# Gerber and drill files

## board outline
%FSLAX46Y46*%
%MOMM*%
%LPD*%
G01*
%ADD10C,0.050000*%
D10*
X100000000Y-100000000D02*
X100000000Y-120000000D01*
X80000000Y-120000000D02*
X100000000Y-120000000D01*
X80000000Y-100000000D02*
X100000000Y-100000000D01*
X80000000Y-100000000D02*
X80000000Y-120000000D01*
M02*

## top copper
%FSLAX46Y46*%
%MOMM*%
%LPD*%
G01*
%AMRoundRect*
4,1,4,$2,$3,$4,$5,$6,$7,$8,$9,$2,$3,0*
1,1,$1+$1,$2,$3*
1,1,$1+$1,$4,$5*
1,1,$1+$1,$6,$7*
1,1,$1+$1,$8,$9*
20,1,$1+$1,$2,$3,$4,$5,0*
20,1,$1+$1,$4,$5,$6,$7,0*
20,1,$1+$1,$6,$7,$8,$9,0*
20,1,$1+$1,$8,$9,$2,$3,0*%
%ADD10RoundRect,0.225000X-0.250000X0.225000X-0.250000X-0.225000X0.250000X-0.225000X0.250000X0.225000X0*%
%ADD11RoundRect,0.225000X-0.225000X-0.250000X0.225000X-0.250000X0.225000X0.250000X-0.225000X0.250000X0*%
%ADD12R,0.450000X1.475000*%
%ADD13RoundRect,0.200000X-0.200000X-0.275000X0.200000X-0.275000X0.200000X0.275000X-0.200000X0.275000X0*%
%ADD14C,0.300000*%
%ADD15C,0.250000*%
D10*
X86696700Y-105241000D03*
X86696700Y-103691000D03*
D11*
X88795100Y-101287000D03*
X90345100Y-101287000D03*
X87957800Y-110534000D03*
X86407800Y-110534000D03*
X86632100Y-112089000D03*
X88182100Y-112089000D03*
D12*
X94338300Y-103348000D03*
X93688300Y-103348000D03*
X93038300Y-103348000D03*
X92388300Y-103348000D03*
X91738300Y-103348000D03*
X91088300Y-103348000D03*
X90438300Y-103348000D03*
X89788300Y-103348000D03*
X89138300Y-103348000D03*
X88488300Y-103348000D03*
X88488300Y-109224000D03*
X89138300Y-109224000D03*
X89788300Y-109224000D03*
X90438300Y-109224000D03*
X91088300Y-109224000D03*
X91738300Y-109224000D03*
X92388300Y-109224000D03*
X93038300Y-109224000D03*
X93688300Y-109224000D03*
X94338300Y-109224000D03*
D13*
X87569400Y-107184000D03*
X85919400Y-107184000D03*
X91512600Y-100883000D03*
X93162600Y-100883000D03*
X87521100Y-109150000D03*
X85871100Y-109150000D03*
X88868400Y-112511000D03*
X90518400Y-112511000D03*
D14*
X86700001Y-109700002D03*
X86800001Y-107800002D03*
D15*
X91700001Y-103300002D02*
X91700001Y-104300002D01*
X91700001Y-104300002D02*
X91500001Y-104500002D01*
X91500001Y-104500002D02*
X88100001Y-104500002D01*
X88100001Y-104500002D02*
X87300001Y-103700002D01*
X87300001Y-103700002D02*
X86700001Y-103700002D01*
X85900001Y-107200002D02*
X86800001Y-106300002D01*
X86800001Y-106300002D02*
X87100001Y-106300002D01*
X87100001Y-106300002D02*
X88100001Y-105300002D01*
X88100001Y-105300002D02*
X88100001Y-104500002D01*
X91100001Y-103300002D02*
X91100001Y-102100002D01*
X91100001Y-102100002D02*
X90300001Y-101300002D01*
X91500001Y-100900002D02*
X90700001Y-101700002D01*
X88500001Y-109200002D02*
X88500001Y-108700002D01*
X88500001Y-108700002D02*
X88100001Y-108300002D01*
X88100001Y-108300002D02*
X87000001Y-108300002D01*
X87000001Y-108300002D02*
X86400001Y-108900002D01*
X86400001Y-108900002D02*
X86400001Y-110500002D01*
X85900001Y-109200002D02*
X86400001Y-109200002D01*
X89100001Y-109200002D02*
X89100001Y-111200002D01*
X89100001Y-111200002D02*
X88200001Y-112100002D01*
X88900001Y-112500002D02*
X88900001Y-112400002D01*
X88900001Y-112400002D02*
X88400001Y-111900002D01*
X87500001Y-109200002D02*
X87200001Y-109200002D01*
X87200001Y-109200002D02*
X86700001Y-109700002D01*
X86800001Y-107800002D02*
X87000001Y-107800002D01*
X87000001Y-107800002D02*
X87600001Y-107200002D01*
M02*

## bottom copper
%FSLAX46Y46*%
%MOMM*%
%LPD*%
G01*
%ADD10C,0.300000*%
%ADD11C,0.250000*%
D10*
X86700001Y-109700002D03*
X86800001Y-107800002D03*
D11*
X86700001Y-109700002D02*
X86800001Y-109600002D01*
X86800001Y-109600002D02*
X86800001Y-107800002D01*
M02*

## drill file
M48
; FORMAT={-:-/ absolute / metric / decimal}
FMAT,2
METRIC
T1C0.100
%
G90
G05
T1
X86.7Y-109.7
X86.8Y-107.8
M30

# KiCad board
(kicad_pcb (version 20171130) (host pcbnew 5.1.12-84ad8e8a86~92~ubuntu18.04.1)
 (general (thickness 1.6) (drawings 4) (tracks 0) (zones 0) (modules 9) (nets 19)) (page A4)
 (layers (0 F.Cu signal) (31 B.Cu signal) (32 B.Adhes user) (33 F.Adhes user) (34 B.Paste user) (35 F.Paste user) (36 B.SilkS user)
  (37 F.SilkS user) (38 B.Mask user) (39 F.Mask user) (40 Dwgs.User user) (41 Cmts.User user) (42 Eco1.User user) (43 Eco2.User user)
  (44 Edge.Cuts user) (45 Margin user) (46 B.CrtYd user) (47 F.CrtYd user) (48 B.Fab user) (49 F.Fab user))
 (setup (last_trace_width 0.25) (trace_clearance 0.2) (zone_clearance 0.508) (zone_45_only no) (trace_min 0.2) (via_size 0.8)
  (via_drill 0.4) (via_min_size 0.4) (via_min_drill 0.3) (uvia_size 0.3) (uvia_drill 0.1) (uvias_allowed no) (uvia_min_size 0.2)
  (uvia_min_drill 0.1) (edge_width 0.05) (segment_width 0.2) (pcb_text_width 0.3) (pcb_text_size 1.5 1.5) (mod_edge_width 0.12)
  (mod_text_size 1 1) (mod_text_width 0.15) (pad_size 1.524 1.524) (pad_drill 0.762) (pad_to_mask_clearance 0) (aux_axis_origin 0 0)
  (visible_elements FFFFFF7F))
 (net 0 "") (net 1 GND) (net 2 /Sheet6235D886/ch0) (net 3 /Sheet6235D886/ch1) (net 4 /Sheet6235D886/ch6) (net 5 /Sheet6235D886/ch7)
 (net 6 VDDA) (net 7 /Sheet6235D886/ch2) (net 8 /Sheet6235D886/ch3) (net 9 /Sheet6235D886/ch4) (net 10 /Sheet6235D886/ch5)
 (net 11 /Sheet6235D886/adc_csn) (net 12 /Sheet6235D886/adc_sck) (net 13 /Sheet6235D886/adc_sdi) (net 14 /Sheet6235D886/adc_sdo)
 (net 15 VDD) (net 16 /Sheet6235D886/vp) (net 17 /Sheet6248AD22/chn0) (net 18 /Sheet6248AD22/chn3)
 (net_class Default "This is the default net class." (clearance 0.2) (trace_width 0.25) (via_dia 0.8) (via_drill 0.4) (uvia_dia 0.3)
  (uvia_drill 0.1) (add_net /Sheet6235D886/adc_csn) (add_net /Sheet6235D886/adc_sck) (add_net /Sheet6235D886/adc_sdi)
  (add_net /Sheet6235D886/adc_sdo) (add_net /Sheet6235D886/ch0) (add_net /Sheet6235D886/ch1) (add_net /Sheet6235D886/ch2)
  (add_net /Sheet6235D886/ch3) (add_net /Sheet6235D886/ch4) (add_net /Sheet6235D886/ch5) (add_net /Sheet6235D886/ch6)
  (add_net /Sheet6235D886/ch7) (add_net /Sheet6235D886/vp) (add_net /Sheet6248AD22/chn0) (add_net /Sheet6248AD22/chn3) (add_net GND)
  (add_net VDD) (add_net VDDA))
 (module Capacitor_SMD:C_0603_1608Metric (layer F.Cu) (at 86.696700 104.466000 270.000000)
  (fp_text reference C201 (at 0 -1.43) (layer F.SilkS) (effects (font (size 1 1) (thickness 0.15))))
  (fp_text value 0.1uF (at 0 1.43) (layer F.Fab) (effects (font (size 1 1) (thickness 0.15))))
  (pad 2 smd roundrect (at 0.775 0 270.000000) (size 0.9 0.95) (layers F.Cu F.Mask F.Paste) (roundrect_rratio 0.25) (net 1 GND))
  (pad 1 smd roundrect (at -0.775 0 270.000000) (size 0.9 0.95) (layers F.Cu F.Mask F.Paste) (roundrect_rratio 0.25)
   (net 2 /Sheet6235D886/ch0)))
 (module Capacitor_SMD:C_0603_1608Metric (layer F.Cu) (at 89.570100 101.287000)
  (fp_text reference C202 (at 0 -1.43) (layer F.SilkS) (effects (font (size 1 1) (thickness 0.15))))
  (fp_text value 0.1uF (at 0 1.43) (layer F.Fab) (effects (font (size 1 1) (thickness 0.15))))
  (pad 1 smd roundrect (at -0.775 0) (size 0.9 0.95) (layers F.Cu F.Mask F.Paste) (roundrect_rratio 0.25) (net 1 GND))
  (pad 2 smd roundrect (at 0.775 0) (size 0.9 0.95) (layers F.Cu F.Mask F.Paste) (roundrect_rratio 0.25) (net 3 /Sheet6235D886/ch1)))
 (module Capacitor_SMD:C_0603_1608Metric (layer F.Cu) (at 87.182800 110.534000)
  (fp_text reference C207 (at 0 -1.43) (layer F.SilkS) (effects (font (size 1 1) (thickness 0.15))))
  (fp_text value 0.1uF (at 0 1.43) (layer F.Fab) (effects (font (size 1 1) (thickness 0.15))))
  (pad 2 smd roundrect (at 0.775 0) (size 0.9 0.95) (layers F.Cu F.Mask F.Paste) (roundrect_rratio 0.25) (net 1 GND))
  (pad 1 smd roundrect (at -0.775 0) (size 0.9 0.95) (layers F.Cu F.Mask F.Paste) (roundrect_rratio 0.25) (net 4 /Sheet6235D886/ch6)))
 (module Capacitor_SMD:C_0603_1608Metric (layer F.Cu) (at 87.407100 112.089000)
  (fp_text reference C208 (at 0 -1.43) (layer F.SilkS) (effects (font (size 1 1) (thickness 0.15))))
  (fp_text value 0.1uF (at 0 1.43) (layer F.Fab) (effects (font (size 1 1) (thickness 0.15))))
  (pad 1 smd roundrect (at -0.775 0) (size 0.9 0.95) (layers F.Cu F.Mask F.Paste) (roundrect_rratio 0.25) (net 1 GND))
  (pad 2 smd roundrect (at 0.775 0) (size 0.9 0.95) (layers F.Cu F.Mask F.Paste) (roundrect_rratio 0.25) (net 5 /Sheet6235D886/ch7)))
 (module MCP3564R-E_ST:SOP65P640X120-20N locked (layer F.Cu) (at 91.413300 106.286000 270.000000)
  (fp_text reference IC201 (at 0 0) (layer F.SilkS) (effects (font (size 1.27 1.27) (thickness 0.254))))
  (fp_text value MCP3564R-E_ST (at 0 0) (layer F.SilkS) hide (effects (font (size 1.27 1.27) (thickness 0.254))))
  (pad 1 smd rect (at -2.938 -2.925) (size 0.45 1.475) (layers F.Cu F.Mask F.Paste) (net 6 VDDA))
  (pad 2 smd rect (at -2.938 -2.275) (size 0.45 1.475) (layers F.Cu F.Mask F.Paste) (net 1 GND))
  (pad 3 smd rect (at -2.938 -1.625) (size 0.45 1.475) (layers F.Cu F.Mask F.Paste) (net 1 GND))
  (pad 4 smd rect (at -2.938 -0.975) (size 0.45 1.475) (layers F.Cu F.Mask F.Paste))
  (pad 5 smd rect (at -2.938 -0.325) (size 0.45 1.475) (layers F.Cu F.Mask F.Paste) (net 2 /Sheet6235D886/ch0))
  (pad 6 smd rect (at -2.938 0.325) (size 0.45 1.475) (layers F.Cu F.Mask F.Paste) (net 3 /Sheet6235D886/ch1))
  (pad 7 smd rect (at -2.938 0.975) (size 0.45 1.475) (layers F.Cu F.Mask F.Paste) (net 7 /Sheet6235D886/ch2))
  (pad 8 smd rect (at -2.938 1.625) (size 0.45 1.475) (layers F.Cu F.Mask F.Paste) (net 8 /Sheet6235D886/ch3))
  (pad 9 smd rect (at -2.938 2.275) (size 0.45 1.475) (layers F.Cu F.Mask F.Paste) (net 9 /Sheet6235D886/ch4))
  (pad 10 smd rect (at -2.938 2.925) (size 0.45 1.475) (layers F.Cu F.Mask F.Paste) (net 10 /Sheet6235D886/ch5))
  (pad 11 smd rect (at 2.938 2.925) (size 0.45 1.475) (layers F.Cu F.Mask F.Paste) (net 4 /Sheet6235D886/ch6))
  (pad 12 smd rect (at 2.938 2.275) (size 0.45 1.475) (layers F.Cu F.Mask F.Paste) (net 5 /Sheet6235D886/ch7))
  (pad 13 smd rect (at 2.938 1.625) (size 0.45 1.475) (layers F.Cu F.Mask F.Paste) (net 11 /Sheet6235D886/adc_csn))
  (pad 14 smd rect (at 2.938 0.975) (size 0.45 1.475) (layers F.Cu F.Mask F.Paste) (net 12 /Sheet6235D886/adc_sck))
  (pad 15 smd rect (at 2.938 0.325) (size 0.45 1.475) (layers F.Cu F.Mask F.Paste) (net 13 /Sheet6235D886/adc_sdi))
  (pad 16 smd rect (at 2.938 -0.325) (size 0.45 1.475) (layers F.Cu F.Mask F.Paste) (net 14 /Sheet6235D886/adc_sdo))
  (pad 17 smd rect (at 2.938 -0.975) (size 0.45 1.475) (layers F.Cu F.Mask F.Paste))
  (pad 18 smd rect (at 2.938 -1.625) (size 0.45 1.475) (layers F.Cu F.Mask F.Paste))
  (pad 19 smd rect (at 2.938 -2.275) (size 0.45 1.475) (layers F.Cu F.Mask F.Paste) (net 1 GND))
  (pad 20 smd rect (at 2.938 -2.925) (size 0.45 1.475) (layers F.Cu F.Mask F.Paste) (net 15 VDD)))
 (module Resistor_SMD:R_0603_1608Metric (layer F.Cu) (at 86.744400 107.184000)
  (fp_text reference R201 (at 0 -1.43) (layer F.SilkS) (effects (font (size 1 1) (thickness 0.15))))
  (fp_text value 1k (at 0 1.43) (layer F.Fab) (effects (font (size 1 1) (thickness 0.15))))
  (pad 2 smd roundrect (at 0.825 0) (size 0.8 0.95) (layers F.Cu F.Mask F.Paste) (roundrect_rratio 0.25) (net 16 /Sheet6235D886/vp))
  (pad 1 smd roundrect (at -0.825 0) (size 0.8 0.95) (layers F.Cu F.Mask F.Paste) (roundrect_rratio 0.25) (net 2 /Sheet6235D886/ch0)))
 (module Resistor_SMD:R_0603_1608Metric (layer F.Cu) (at 92.337600 100.883000)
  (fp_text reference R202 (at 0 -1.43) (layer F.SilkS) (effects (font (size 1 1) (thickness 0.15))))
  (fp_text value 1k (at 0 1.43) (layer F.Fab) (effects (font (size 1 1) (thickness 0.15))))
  (pad 1 smd roundrect (at -0.825 0) (size 0.8 0.95) (layers F.Cu F.Mask F.Paste) (roundrect_rratio 0.25) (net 3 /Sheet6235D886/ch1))
  (pad 2 smd roundrect (at 0.825 0) (size 0.8 0.95) (layers F.Cu F.Mask F.Paste) (roundrect_rratio 0.25) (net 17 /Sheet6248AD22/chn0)))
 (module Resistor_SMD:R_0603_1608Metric (layer F.Cu) (at 86.696100 109.150000)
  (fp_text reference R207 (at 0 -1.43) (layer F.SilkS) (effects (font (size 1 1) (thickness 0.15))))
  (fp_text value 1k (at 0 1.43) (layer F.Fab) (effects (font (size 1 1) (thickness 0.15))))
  (pad 2 smd roundrect (at 0.825 0) (size 0.8 0.95) (layers F.Cu F.Mask F.Paste) (roundrect_rratio 0.25) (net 16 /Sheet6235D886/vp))
  (pad 1 smd roundrect (at -0.825 0) (size 0.8 0.95) (layers F.Cu F.Mask F.Paste) (roundrect_rratio 0.25) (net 4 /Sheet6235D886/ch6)))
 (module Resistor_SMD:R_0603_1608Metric (layer F.Cu) (at 89.693400 112.511000)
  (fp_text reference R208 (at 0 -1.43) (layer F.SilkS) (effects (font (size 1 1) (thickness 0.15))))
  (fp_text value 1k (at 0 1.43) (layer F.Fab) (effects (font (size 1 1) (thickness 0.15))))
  (pad 1 smd roundrect (at -0.825 0) (size 0.8 0.95) (layers F.Cu F.Mask F.Paste) (roundrect_rratio 0.25) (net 5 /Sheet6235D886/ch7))
  (pad 2 smd roundrect (at 0.825 0) (size 0.8 0.95) (layers F.Cu F.Mask F.Paste) (roundrect_rratio 0.25) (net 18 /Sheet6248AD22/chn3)))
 (gr_line (start 100 100) (end 100 120) (layer Edge.Cuts) (width 0.05))
 (gr_line (start 80 120) (end 100 120) (layer Edge.Cuts) (width 0.05))
 (gr_line (start 80 100) (end 100 100) (layer Edge.Cuts) (width 0.05))
 (gr_line (start 80 100) (end 80 120) (layer Edge.Cuts) (width 0.05))
 (segment (start 91.700001 103.300002) (end 91.700001 104.300002) (width 0.250000) (layer F.Cu) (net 2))
 (segment (start 91.700001 104.300002) (end 91.500001 104.500002) (width 0.250000) (layer F.Cu) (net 2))
 (segment (start 91.500001 104.500002) (end 88.100001 104.500002) (width 0.250000) (layer F.Cu) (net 2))
 (segment (start 88.100001 104.500002) (end 87.300001 103.700002) (width 0.250000) (layer F.Cu) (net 2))
 (segment (start 87.300001 103.700002) (end 86.700001 103.700002) (width 0.250000) (layer F.Cu) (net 2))
 (segment (start 85.900001 107.200002) (end 86.800001 106.300002) (width 0.250000) (layer F.Cu) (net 2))
 (segment (start 86.800001 106.300002) (end 87.100001 106.300002) (width 0.250000) (layer F.Cu) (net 2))
 (segment (start 87.100001 106.300002) (end 88.100001 105.300002) (width 0.250000) (layer F.Cu) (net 2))
 (segment (start 88.100001 105.300002) (end 88.100001 104.500002) (width 0.250000) (layer F.Cu) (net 2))
 (segment (start 91.100001 103.300002) (end 91.100001 102.100002) (width 0.250000) (layer F.Cu) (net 3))
 (segment (start 91.100001 102.100002) (end 90.300001 101.300002) (width 0.250000) (layer F.Cu) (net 3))
 (segment (start 91.500001 100.900002) (end 90.700001 101.700002) (width 0.250000) (layer F.Cu) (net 3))
 (segment (start 88.500001 109.200002) (end 88.500001 108.700002) (width 0.250000) (layer F.Cu) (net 4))
 (segment (start 88.500001 108.700002) (end 88.100001 108.300002) (width 0.250000) (layer F.Cu) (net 4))
 (segment (start 88.100001 108.300002) (end 87.000001 108.300002) (width 0.250000) (layer F.Cu) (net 4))
 (segment (start 87.000001 108.300002) (end 86.400001 108.900002) (width 0.250000) (layer F.Cu) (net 4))
 (segment (start 86.400001 108.900002) (end 86.400001 110.500002) (width 0.250000) (layer F.Cu) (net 4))
 (segment (start 85.900001 109.200002) (end 86.400001 109.200002) (width 0.250000) (layer F.Cu) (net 4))
 (segment (start 89.100001 109.200002) (end 89.100001 111.200002) (width 0.250000) (layer F.Cu) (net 5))
 (segment (start 89.100001 111.200002) (end 88.200001 112.100002) (width 0.250000) (layer F.Cu) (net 5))
 (segment (start 88.900001 112.500002) (end 88.900001 112.400002) (width 0.250000) (layer F.Cu) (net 5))
 (segment (start 88.900001 112.400002) (end 88.400001 111.900002) (width 0.250000) (layer F.Cu) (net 5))
 (segment (start 87.500001 109.200002) (end 87.200001 109.200002) (width 0.250000) (layer F.Cu) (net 16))
 (segment (start 87.200001 109.200002) (end 86.700001 109.700002) (width 0.250000) (layer F.Cu) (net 16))
 (segment (start 86.700001 109.700002) (end 86.800001 109.600002) (width 0.250000) (layer B.Cu) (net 16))
 (segment (start 86.800001 109.600002) (end 86.800001 107.800002) (width 0.250000) (layer B.Cu) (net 16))
 (segment (start 86.800001 107.800002) (end 87.000001 107.800002) (width 0.250000) (layer F.Cu) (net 16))
 (segment (start 87.000001 107.800002) (end 87.600001 107.200002) (width 0.250000) (layer F.Cu) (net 16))
 (via micro (at 86.700001 109.700002) (size 0.300000) (drill 0.100000) (layers F.Cu B.Cu) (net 16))
 (via micro (at 86.800001 107.800002) (size 0.300000) (drill 0.100000) (layers F.Cu B.Cu) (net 16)))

